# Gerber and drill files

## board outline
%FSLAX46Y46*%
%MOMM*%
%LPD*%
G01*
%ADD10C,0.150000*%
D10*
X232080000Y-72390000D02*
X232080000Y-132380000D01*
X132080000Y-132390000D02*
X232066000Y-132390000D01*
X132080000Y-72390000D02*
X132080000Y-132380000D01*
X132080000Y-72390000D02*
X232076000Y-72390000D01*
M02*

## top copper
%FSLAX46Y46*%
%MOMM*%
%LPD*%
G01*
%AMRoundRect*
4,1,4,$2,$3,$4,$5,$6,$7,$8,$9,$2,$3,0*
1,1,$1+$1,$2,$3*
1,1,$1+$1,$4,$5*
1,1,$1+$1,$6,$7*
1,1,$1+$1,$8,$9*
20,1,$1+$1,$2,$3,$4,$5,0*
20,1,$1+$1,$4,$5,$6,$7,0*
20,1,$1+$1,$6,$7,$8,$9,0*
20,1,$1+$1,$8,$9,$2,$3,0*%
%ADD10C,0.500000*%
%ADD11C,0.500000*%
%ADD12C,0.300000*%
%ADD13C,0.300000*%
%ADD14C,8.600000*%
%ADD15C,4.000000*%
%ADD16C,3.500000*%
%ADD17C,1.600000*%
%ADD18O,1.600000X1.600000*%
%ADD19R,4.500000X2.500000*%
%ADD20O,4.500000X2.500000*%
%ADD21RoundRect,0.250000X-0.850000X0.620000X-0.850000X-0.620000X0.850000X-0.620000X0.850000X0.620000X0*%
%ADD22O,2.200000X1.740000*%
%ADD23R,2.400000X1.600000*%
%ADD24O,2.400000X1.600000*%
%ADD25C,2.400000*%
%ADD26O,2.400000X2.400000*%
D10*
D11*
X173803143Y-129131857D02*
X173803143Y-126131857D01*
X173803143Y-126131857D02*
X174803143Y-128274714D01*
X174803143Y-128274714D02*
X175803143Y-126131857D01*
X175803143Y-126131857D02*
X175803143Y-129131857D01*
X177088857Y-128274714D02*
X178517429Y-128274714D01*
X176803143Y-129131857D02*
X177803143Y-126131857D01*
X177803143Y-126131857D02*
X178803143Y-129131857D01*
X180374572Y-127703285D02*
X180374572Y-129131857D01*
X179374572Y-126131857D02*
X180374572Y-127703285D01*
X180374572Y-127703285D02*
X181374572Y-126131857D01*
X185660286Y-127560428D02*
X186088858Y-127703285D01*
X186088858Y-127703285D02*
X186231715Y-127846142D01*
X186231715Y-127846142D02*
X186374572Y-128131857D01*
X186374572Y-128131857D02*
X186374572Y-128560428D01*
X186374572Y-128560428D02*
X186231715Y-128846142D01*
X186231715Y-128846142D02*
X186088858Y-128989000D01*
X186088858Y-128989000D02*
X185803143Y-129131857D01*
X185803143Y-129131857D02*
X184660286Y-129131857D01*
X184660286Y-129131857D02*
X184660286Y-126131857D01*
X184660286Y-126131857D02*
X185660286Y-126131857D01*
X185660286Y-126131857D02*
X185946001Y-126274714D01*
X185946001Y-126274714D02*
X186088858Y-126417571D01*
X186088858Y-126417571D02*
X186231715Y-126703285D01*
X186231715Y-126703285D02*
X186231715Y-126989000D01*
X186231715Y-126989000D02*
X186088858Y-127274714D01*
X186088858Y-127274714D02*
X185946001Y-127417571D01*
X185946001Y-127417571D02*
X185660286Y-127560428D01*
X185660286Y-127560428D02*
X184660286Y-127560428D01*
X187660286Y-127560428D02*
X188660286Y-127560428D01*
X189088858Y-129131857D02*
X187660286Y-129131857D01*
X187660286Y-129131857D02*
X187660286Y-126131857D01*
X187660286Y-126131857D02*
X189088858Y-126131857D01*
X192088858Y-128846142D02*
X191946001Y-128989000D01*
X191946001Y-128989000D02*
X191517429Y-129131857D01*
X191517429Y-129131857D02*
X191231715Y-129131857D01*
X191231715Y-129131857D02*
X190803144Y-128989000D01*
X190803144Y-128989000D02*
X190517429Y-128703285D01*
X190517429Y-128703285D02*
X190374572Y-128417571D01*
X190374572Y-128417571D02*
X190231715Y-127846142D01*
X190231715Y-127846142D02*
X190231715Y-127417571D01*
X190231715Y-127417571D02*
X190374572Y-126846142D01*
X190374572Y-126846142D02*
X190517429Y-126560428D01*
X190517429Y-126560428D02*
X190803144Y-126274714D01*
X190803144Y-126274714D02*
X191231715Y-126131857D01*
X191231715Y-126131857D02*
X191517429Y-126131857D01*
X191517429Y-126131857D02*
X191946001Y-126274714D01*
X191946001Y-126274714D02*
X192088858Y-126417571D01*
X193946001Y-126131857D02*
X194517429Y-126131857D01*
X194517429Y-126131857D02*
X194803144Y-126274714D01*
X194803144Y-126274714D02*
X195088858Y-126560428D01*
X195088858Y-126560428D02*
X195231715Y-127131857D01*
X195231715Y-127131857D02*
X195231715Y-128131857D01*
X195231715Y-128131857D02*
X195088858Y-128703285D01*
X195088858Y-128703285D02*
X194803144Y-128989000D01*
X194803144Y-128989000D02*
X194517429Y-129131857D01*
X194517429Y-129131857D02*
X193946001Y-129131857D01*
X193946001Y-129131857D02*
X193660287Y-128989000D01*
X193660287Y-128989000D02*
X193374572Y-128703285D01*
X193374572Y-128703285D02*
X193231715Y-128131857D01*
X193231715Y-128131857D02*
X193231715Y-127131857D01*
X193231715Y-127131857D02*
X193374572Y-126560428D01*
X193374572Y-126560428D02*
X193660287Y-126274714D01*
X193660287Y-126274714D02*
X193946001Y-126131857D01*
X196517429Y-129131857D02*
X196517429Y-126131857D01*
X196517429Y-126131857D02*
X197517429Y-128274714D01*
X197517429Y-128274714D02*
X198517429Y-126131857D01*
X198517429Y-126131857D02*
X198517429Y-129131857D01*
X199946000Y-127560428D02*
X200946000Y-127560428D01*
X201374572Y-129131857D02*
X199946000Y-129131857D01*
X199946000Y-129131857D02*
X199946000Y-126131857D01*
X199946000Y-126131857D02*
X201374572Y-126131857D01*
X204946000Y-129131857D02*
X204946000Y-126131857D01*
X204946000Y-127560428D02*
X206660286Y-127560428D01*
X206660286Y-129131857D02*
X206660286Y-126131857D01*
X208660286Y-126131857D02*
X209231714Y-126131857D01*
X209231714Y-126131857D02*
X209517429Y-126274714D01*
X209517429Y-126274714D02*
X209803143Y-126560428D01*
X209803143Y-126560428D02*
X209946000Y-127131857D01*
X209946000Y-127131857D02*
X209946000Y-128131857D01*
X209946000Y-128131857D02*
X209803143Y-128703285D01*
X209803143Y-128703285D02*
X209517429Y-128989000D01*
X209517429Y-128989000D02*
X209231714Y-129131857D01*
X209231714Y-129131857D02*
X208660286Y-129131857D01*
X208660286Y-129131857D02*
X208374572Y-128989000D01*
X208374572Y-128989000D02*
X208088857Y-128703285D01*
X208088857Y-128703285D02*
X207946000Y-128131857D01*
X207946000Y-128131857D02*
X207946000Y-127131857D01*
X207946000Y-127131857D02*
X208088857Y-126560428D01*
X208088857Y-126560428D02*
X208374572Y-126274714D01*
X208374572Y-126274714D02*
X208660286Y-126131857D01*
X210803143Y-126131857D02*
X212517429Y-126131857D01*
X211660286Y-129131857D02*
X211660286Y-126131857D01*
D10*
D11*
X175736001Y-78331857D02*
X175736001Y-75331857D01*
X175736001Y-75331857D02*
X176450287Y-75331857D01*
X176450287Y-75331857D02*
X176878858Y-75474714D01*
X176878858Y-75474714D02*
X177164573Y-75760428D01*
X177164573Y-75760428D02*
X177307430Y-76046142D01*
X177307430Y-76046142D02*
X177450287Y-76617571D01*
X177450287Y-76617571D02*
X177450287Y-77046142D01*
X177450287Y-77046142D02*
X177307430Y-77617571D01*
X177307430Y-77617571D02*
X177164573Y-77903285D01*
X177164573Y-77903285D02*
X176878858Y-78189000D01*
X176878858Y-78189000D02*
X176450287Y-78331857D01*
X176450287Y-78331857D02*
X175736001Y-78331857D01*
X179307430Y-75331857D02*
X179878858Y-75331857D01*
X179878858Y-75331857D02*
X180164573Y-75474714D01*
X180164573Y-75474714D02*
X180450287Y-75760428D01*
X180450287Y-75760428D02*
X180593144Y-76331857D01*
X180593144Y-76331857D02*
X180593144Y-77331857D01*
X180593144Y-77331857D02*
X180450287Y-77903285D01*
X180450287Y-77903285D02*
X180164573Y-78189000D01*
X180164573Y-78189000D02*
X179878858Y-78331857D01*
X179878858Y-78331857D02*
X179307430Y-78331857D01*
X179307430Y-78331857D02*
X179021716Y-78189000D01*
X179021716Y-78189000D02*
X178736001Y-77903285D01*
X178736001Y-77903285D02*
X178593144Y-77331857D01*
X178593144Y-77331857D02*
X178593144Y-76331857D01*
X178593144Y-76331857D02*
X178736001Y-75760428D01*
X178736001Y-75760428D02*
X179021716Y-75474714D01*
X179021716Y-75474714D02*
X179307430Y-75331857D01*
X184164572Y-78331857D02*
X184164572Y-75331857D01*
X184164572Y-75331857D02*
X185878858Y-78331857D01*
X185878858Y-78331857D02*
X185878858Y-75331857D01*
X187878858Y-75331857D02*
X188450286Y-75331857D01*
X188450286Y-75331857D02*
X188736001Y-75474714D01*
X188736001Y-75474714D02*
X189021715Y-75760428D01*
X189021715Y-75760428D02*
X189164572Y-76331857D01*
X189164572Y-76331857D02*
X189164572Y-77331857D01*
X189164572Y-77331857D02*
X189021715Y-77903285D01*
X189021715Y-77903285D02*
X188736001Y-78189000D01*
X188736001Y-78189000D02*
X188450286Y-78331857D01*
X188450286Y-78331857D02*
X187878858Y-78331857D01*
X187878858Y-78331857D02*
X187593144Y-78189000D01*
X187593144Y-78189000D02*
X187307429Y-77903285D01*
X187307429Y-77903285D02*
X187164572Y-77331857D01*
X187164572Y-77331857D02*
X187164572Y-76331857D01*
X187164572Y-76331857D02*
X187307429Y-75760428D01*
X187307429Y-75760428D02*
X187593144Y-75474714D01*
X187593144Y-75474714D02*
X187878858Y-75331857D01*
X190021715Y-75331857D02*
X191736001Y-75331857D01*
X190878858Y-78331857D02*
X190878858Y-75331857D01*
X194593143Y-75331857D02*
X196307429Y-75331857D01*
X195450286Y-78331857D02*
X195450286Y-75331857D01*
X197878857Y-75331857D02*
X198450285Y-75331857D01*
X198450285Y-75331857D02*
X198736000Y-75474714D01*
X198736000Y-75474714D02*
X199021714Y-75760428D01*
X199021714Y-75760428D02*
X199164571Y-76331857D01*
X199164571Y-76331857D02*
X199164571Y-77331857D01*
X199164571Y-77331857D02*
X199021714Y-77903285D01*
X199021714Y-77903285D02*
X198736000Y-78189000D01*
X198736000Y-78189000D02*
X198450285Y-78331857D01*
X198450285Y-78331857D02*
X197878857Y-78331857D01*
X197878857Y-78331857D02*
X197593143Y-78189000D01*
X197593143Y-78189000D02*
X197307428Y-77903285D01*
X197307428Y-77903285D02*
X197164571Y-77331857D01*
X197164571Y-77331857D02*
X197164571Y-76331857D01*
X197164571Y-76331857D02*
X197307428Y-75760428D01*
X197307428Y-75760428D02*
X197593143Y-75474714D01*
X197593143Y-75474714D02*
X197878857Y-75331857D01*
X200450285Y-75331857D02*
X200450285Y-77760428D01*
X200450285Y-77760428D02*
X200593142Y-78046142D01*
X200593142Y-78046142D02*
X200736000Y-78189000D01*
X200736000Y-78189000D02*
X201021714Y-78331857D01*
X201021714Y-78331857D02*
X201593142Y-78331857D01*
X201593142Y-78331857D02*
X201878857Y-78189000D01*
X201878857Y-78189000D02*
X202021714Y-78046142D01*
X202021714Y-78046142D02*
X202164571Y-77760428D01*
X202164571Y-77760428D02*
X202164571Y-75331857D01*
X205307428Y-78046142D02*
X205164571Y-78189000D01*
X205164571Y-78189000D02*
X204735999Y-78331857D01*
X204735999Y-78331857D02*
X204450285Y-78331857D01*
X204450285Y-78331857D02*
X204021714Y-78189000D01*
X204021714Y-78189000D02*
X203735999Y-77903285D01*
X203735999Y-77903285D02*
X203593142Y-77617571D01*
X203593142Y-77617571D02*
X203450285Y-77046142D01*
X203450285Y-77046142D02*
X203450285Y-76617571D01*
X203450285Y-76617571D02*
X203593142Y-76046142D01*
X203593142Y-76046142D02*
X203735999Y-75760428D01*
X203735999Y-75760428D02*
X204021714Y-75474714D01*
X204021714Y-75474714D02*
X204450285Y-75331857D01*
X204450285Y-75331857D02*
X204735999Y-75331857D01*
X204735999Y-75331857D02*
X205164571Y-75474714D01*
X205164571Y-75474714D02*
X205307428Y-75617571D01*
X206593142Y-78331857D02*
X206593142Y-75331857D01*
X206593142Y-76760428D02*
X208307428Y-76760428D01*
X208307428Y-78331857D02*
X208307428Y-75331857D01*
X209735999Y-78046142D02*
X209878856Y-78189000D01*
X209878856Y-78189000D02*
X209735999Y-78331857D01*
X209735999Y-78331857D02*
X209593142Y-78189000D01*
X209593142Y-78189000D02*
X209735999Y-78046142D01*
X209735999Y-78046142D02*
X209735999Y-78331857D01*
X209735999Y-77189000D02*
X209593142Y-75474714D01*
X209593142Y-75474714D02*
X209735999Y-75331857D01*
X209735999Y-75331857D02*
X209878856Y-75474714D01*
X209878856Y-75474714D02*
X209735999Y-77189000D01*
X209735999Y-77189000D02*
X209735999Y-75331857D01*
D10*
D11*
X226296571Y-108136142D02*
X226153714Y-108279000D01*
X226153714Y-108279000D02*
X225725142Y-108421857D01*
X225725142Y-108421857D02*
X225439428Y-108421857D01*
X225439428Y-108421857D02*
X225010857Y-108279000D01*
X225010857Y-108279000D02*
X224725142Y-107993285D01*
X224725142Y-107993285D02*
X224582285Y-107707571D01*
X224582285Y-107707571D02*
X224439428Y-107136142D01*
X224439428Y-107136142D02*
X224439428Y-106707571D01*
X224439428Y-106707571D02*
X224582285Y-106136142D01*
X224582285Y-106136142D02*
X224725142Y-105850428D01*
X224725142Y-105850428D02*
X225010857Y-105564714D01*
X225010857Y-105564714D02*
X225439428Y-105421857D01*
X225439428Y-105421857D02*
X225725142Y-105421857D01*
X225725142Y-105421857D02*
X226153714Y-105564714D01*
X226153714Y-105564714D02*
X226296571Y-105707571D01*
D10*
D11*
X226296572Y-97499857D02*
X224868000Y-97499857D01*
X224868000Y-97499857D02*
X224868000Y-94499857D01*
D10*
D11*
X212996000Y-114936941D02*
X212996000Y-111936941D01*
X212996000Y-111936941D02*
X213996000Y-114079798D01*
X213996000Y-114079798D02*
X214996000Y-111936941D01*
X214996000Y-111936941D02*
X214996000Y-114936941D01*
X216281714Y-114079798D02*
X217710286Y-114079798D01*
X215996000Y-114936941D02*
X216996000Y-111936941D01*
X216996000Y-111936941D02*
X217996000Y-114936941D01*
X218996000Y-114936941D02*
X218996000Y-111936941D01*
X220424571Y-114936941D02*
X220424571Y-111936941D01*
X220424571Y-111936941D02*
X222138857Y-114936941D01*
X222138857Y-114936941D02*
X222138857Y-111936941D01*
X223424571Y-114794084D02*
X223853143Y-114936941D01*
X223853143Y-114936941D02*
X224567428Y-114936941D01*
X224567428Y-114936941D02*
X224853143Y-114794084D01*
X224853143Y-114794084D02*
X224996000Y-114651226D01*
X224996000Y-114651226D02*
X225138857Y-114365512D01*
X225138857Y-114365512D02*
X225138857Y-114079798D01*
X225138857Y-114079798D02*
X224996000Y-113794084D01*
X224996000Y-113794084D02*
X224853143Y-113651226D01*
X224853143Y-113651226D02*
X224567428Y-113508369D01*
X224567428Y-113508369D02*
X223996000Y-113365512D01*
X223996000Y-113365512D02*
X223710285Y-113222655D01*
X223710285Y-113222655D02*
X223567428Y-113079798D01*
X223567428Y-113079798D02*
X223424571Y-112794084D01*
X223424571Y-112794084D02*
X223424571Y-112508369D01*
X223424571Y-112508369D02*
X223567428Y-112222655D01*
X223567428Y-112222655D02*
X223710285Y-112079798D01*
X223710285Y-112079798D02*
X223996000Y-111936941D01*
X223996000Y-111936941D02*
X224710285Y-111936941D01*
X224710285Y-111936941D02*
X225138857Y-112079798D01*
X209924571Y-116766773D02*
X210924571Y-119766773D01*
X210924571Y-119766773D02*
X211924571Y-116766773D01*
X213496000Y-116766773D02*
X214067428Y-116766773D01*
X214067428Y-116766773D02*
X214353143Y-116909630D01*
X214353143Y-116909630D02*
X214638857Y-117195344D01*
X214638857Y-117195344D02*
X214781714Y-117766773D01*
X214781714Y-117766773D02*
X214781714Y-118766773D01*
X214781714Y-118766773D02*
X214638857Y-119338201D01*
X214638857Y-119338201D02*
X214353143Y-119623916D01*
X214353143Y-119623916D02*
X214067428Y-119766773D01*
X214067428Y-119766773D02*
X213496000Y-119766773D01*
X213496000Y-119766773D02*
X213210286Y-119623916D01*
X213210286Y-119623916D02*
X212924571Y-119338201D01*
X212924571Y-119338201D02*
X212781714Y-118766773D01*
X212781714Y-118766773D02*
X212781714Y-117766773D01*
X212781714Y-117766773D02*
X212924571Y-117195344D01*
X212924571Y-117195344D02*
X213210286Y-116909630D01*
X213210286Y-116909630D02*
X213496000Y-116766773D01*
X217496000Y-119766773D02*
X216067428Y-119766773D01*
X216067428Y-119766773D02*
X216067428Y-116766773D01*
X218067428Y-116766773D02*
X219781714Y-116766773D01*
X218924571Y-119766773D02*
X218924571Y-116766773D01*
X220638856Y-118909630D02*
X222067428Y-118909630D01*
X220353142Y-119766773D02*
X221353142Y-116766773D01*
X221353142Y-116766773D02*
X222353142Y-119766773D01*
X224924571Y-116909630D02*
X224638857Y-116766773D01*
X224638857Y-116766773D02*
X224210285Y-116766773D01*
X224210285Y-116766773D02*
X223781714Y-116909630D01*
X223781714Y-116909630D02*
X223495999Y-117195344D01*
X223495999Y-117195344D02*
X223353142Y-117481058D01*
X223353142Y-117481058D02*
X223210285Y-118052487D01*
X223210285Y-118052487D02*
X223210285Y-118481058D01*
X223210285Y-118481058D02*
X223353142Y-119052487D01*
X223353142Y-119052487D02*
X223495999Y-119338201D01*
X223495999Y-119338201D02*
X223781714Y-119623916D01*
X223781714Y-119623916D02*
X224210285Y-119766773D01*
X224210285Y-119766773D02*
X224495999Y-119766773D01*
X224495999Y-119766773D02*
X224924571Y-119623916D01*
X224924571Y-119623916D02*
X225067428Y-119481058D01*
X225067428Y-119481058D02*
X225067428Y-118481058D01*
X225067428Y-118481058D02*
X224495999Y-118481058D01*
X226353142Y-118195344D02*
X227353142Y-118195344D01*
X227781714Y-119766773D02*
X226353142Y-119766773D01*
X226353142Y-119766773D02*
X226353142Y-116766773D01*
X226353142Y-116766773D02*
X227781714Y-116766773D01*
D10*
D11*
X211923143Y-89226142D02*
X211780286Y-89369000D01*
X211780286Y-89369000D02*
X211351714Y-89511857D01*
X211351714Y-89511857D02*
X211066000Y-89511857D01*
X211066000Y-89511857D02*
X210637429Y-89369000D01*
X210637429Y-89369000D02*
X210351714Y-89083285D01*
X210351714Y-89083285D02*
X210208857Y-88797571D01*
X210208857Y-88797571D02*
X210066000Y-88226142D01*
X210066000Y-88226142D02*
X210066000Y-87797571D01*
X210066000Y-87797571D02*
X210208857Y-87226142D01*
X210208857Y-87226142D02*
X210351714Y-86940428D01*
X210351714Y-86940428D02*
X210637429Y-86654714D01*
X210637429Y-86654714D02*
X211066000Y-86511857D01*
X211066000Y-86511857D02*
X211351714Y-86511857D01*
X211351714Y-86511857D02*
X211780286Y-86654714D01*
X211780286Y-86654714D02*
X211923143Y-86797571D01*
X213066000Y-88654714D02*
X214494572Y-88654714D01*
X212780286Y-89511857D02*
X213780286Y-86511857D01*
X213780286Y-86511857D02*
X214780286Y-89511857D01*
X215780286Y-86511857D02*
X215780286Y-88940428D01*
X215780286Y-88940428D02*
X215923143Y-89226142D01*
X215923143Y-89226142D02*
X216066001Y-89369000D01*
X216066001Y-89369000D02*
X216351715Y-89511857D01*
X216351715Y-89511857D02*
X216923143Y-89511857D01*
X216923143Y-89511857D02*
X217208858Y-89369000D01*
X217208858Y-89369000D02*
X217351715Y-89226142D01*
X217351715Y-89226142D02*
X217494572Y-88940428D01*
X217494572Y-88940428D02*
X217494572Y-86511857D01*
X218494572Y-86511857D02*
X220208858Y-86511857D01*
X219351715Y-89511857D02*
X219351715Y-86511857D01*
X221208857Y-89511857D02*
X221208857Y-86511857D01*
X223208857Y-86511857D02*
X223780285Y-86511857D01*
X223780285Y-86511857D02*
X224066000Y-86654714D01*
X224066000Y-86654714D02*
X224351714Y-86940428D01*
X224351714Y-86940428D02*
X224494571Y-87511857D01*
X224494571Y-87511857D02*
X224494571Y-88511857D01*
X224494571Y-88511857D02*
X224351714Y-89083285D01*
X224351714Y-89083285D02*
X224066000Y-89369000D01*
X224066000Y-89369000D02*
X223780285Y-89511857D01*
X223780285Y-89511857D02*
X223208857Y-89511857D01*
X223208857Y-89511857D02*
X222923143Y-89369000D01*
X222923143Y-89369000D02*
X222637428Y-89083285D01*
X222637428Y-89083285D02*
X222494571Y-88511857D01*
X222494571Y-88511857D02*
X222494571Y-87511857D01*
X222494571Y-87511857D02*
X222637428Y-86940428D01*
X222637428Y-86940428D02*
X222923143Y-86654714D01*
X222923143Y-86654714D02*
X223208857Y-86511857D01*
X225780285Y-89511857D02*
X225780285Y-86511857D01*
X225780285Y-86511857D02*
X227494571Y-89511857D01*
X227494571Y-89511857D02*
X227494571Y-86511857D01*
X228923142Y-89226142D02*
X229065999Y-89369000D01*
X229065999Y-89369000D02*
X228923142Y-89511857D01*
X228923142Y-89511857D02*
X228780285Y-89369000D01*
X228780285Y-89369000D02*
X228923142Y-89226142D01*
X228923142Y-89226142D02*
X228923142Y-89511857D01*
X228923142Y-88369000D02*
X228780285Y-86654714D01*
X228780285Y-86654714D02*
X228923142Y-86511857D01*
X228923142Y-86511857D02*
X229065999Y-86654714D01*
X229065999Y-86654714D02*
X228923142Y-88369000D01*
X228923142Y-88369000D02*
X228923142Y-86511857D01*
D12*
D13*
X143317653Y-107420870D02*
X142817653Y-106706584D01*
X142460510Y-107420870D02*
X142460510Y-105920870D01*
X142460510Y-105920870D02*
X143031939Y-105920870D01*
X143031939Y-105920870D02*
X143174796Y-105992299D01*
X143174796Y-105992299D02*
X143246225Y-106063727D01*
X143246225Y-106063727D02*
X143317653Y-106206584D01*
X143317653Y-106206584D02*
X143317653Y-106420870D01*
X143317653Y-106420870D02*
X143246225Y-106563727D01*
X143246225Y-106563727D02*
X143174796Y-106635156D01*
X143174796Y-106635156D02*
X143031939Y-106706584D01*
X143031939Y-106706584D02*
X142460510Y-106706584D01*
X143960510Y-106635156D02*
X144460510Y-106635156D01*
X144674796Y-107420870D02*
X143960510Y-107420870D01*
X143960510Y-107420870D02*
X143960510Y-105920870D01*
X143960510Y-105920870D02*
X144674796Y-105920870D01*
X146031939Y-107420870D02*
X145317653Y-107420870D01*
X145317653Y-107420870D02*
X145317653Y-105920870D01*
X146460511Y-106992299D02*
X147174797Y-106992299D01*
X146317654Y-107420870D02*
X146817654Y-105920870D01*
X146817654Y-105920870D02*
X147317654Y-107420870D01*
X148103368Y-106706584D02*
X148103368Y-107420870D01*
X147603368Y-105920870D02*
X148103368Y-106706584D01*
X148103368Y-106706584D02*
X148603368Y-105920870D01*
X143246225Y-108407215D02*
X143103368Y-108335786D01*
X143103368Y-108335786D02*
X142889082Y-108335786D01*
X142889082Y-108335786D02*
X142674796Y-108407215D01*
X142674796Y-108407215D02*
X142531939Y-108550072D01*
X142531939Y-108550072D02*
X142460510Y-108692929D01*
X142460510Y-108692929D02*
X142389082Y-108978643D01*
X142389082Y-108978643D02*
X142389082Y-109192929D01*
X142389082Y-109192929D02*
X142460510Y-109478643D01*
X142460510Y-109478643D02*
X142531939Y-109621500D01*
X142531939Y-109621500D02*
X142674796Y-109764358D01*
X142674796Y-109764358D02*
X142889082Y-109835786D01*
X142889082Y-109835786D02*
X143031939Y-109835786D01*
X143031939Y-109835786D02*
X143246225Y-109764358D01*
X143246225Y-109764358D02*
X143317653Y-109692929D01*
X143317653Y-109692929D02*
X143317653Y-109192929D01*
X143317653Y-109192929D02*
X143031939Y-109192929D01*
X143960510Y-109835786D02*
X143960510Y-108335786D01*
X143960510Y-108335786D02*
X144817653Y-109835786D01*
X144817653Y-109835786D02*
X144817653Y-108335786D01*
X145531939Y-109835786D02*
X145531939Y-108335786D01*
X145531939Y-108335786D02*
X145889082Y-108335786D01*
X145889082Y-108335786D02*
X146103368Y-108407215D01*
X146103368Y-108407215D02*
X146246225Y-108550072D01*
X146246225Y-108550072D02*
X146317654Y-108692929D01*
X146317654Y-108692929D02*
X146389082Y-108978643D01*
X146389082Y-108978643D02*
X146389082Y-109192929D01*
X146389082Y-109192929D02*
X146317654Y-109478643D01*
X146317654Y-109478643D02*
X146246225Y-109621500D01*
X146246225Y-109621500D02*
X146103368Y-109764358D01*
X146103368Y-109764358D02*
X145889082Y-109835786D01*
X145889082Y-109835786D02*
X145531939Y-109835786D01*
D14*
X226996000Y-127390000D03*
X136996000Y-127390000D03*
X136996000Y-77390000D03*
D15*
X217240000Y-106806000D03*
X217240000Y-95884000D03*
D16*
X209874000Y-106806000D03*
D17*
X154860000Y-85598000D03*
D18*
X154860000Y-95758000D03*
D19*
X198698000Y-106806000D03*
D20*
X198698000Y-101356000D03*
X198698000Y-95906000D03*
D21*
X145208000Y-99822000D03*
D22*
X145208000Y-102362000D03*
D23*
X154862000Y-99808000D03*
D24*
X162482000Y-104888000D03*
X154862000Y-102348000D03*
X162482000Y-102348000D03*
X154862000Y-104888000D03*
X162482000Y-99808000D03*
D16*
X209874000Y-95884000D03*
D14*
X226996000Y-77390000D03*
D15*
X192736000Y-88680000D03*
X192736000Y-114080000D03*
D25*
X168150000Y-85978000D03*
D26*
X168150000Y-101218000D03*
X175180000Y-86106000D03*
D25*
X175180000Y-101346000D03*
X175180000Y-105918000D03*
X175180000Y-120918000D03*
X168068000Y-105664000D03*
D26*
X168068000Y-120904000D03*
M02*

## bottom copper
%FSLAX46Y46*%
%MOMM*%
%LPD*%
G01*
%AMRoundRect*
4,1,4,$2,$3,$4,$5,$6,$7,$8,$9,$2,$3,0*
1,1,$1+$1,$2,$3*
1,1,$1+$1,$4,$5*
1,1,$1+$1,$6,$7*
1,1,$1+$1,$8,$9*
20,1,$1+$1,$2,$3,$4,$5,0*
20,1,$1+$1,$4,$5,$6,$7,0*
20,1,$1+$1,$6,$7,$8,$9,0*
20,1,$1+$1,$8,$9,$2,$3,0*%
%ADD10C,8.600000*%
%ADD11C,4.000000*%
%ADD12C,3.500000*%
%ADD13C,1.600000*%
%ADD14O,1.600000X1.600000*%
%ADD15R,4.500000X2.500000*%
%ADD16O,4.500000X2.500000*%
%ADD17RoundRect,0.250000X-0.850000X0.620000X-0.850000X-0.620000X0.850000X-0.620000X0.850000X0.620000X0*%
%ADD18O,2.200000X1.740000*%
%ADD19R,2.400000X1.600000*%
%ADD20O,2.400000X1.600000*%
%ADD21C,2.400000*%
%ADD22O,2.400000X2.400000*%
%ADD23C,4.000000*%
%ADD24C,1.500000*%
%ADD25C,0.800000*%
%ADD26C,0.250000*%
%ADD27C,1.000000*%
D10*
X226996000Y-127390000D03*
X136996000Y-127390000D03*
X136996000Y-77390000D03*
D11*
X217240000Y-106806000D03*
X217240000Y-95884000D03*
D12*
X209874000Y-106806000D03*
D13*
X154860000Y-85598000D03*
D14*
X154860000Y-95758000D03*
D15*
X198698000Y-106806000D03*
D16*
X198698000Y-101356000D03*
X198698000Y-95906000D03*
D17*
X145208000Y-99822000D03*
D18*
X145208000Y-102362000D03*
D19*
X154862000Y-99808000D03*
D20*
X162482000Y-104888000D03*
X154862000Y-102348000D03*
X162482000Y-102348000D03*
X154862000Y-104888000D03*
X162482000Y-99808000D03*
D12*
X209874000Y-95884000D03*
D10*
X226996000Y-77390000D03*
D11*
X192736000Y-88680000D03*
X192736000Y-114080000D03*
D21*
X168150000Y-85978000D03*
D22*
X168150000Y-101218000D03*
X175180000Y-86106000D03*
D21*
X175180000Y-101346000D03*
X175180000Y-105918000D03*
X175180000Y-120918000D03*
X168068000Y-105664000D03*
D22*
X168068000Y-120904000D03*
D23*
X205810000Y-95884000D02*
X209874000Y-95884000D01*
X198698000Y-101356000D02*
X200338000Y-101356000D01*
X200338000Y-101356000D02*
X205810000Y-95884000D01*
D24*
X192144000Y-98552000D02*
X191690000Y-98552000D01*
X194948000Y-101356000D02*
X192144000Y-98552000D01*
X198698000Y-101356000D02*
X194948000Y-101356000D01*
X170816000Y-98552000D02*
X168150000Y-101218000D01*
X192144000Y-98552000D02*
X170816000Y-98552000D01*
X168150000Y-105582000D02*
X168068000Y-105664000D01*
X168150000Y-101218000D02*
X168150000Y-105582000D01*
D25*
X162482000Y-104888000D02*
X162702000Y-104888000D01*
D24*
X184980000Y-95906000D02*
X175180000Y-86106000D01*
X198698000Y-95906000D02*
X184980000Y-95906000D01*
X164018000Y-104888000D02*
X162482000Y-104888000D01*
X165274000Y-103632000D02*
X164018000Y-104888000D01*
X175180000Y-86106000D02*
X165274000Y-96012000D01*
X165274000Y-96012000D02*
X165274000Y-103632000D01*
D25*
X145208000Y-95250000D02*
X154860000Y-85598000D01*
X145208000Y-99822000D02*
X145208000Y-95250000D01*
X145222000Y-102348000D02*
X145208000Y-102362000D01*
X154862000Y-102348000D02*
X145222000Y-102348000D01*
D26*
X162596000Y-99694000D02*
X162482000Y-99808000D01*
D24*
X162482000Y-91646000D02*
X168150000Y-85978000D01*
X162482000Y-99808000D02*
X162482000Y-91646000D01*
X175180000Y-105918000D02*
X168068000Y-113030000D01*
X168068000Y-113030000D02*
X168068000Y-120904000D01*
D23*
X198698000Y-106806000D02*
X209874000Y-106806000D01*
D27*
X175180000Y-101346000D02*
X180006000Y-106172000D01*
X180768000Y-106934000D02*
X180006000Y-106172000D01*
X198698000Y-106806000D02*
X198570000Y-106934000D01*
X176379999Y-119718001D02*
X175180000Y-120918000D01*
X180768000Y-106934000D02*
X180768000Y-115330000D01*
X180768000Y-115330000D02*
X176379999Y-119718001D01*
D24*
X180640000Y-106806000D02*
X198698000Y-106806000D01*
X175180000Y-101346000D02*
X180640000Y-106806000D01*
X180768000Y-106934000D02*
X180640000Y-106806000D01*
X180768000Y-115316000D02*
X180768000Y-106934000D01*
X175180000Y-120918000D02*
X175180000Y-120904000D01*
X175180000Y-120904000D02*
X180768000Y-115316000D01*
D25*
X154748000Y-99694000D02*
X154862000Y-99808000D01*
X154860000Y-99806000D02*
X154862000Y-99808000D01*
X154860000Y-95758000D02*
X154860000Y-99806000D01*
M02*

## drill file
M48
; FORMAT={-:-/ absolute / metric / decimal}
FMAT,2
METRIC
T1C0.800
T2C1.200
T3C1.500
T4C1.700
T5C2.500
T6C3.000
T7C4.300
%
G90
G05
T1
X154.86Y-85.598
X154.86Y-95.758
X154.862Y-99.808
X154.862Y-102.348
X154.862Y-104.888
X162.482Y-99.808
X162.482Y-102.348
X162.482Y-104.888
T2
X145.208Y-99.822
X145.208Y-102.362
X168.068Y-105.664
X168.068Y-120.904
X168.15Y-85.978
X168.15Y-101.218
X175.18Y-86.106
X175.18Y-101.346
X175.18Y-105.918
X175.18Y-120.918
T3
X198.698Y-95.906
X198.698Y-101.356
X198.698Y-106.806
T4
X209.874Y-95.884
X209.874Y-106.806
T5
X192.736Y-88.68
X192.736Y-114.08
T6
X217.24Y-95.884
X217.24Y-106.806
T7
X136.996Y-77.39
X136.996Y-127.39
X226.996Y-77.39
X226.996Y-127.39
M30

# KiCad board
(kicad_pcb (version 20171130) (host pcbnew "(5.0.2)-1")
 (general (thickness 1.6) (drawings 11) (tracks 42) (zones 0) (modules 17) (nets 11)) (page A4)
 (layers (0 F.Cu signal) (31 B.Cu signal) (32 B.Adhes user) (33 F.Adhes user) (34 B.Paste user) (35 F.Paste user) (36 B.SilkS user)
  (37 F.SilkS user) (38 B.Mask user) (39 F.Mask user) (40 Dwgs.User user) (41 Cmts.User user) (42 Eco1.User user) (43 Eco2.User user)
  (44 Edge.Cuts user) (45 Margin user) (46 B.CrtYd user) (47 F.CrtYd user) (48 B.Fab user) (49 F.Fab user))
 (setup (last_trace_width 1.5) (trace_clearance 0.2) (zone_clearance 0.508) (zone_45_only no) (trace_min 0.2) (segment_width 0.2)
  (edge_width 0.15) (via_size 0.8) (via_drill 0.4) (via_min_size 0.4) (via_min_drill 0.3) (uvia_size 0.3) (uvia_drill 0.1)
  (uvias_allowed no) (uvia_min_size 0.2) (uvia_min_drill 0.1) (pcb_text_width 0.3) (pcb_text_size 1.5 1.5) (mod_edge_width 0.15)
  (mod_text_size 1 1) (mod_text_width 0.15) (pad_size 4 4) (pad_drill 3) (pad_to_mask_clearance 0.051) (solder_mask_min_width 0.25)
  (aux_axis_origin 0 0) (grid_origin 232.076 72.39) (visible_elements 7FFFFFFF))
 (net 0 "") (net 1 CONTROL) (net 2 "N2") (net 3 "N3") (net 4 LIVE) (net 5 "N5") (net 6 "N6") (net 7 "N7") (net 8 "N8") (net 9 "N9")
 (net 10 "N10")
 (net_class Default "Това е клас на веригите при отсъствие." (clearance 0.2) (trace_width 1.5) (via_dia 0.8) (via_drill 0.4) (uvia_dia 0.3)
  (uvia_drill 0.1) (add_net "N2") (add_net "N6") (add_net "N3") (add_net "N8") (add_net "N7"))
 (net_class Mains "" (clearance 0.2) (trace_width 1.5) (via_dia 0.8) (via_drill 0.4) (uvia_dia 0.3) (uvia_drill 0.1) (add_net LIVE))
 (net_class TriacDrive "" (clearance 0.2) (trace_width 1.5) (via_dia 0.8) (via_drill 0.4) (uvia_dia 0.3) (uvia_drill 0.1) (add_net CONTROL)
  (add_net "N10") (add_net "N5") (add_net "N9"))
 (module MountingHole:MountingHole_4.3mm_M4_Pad (layer F.Cu) (at 226.996 127.39)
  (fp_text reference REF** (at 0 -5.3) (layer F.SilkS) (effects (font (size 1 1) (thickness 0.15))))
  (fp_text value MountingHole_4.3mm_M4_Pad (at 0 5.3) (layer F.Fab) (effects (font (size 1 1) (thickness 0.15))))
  (pad 1 thru_hole circle (at 0 0) (size 8.6 8.6) (drill 4.3) (layers *.Cu *.Mask)))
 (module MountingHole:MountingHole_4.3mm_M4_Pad (layer F.Cu) (at 136.996 127.39)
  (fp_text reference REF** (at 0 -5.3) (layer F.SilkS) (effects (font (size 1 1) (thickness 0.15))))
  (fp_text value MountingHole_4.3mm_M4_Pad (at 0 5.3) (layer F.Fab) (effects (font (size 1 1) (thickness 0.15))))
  (pad 1 thru_hole circle (at 0 0) (size 8.6 8.6) (drill 4.3) (layers *.Cu *.Mask)))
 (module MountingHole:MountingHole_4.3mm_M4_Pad (layer F.Cu) (at 136.996 77.39)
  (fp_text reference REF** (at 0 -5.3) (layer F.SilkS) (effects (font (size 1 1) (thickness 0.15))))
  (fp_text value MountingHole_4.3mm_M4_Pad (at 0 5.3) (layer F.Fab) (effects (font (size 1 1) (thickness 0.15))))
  (pad 1 thru_hole circle (at 0 0) (size 8.6 8.6) (drill 4.3) (layers *.Cu *.Mask)))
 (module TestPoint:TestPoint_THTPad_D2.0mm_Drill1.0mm (layer F.Cu) (at 217.24 106.806)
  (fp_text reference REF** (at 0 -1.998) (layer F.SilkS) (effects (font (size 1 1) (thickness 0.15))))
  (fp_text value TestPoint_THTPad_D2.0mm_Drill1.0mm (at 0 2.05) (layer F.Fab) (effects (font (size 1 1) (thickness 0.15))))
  (pad 1 thru_hole circle (at 0 0) (size 4 4) (drill 3) (layers *.Cu *.Mask)))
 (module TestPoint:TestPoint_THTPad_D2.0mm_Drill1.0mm (layer F.Cu) (at 217.24 95.884)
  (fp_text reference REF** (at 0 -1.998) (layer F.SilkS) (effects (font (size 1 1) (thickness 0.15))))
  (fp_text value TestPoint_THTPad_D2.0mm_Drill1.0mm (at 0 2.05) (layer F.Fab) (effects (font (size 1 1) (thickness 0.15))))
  (pad 1 thru_hole circle (at 0 0) (size 4 4) (drill 3) (layers *.Cu *.Mask)))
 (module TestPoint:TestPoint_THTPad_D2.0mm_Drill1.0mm (layer F.Cu) (at 209.874 106.806)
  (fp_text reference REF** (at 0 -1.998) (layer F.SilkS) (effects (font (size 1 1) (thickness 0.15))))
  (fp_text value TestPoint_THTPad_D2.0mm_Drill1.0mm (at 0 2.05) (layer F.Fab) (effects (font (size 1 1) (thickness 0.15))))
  (pad 1 thru_hole circle (at 0 0) (size 3.5 3.5) (drill 1.7) (layers *.Cu *.Mask) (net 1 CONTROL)))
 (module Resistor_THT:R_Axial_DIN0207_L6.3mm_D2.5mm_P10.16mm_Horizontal (layer F.Cu) (at 154.86 85.598 270)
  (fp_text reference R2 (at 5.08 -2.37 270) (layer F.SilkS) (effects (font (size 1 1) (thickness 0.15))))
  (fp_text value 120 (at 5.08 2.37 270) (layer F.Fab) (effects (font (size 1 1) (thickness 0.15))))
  (pad 1 thru_hole circle (at 0 0 270) (size 1.6 1.6) (drill 0.8) (layers *.Cu *.Mask) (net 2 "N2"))
  (pad 2 thru_hole oval (at 10.16 0 270) (size 1.6 1.6) (drill 0.8) (layers *.Cu *.Mask) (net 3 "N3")))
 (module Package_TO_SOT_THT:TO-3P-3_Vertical (layer F.Cu) (at 198.698 106.806 90)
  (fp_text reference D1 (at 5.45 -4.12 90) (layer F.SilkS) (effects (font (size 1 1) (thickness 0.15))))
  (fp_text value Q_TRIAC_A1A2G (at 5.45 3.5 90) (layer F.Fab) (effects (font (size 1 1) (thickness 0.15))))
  (pad 1 thru_hole rect (at 0 0 90) (size 2.5 4.5) (drill 1.5) (layers *.Cu *.Mask) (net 1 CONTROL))
  (pad 2 thru_hole oval (at 5.45 0 90) (size 2.5 4.5) (drill 1.5) (layers *.Cu *.Mask) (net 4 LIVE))
  (pad 3 thru_hole oval (at 10.9 0 90) (size 2.5 4.5) (drill 1.5) (layers *.Cu *.Mask) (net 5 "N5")))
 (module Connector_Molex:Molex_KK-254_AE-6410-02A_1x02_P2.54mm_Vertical (layer F.Cu) (at 145.208 99.822 270)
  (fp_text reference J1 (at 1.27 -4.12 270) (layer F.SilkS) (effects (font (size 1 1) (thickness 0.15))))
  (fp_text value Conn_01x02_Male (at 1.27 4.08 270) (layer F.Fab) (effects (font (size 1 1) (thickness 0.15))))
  (pad 1 thru_hole roundrect (at 0 0 270) (size 1.74 2.2) (drill 1.2) (layers *.Cu *.Mask) (roundrect_rratio 0.143678) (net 2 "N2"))
  (pad 2 thru_hole oval (at 2.54 0 270) (size 1.74 2.2) (drill 1.2) (layers *.Cu *.Mask) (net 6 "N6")))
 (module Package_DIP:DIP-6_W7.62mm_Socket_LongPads (layer F.Cu) (at 154.862 99.808)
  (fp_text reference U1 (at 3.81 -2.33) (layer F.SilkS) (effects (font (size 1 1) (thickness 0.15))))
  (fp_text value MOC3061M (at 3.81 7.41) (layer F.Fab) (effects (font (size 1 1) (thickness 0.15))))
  (pad 1 thru_hole rect (at 0 0) (size 2.4 1.6) (drill 0.8) (layers *.Cu *.Mask) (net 3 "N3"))
  (pad 4 thru_hole oval (at 7.62 5.08) (size 2.4 1.6) (drill 0.8) (layers *.Cu *.Mask) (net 5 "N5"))
  (pad 2 thru_hole oval (at 0 2.54) (size 2.4 1.6) (drill 0.8) (layers *.Cu *.Mask) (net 6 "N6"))
  (pad 5 thru_hole oval (at 7.62 2.54) (size 2.4 1.6) (drill 0.8) (layers *.Cu *.Mask) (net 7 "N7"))
  (pad 3 thru_hole oval (at 0 5.08) (size 2.4 1.6) (drill 0.8) (layers *.Cu *.Mask) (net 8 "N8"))
  (pad 6 thru_hole oval (at 7.62 0) (size 2.4 1.6) (drill 0.8) (layers *.Cu *.Mask) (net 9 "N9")))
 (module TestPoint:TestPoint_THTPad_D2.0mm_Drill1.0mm (layer F.Cu) (at 209.874 95.884)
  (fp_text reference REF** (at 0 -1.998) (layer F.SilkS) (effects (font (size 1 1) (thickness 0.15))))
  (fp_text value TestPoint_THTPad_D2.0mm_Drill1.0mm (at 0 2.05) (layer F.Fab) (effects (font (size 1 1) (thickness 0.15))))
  (pad 1 thru_hole circle (at 0 0) (size 3.5 3.5) (drill 1.7) (layers *.Cu *.Mask) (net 4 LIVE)))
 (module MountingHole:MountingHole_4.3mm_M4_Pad (layer F.Cu) (at 226.996 77.39)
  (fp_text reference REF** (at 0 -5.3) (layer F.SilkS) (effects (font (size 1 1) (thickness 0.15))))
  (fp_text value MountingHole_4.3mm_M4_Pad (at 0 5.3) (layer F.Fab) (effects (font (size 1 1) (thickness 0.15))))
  (pad 1 thru_hole circle (at 0 0) (size 8.6 8.6) (drill 4.3) (layers *.Cu *.Mask)))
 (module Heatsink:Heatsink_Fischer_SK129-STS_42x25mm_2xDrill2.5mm (layer F.Cu) (at 192.736 101.38 90)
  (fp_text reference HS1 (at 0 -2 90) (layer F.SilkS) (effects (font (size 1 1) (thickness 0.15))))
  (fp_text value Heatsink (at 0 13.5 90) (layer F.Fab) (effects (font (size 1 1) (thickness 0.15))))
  (pad 1 thru_hole circle (at 12.7 0 90) (size 4 4) (drill 2.5) (layers *.Cu *.Mask))
  (pad 1 thru_hole circle (at -12.7 0 270) (size 4 4) (drill 2.5) (layers *.Cu *.Mask)))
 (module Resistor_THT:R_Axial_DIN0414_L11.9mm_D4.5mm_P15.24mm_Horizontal (layer F.Cu) (at 168.15 85.978 270)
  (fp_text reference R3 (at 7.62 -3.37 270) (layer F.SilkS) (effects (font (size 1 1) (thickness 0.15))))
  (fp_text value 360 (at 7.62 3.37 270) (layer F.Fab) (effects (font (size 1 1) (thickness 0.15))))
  (pad 1 thru_hole circle (at 0 0 270) (size 2.4 2.4) (drill 1.2) (layers *.Cu *.Mask) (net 9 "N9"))
  (pad 2 thru_hole oval (at 15.24 0 270) (size 2.4 2.4) (drill 1.2) (layers *.Cu *.Mask) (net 4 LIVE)))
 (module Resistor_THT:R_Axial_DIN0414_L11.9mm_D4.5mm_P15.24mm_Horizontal (layer F.Cu) (at 175.18 101.346 90)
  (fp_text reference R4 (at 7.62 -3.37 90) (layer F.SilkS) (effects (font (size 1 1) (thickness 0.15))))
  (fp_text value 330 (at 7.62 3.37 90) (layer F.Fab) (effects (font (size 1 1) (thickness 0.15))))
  (pad 2 thru_hole oval (at 15.24 0 90) (size 2.4 2.4) (drill 1.2) (layers *.Cu *.Mask) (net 5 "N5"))
  (pad 1 thru_hole circle (at 0 0 90) (size 2.4 2.4) (drill 1.2) (layers *.Cu *.Mask) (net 1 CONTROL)))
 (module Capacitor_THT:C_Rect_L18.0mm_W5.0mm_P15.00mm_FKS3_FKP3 (layer F.Cu) (at 175.18 105.918 270)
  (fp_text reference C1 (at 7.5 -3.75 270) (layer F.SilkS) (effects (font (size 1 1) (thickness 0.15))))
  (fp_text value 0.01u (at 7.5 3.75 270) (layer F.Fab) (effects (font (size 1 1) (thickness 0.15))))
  (pad 1 thru_hole circle (at 0 0 270) (size 2.4 2.4) (drill 1.2) (layers *.Cu *.Mask) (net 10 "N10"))
  (pad 2 thru_hole circle (at 15 0 270) (size 2.4 2.4) (drill 1.2) (layers *.Cu *.Mask) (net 1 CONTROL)))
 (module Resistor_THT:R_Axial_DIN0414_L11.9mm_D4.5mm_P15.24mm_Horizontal (layer F.Cu) (at 168.068 105.664 270)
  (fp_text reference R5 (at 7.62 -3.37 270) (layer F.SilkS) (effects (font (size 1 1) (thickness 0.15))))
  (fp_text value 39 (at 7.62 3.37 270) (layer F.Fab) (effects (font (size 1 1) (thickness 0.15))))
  (pad 1 thru_hole circle (at 0 0 270) (size 2.4 2.4) (drill 1.2) (layers *.Cu *.Mask) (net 4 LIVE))
  (pad 2 thru_hole oval (at 15.24 0 270) (size 2.4 2.4) (drill 1.2) (layers *.Cu *.Mask) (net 10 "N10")))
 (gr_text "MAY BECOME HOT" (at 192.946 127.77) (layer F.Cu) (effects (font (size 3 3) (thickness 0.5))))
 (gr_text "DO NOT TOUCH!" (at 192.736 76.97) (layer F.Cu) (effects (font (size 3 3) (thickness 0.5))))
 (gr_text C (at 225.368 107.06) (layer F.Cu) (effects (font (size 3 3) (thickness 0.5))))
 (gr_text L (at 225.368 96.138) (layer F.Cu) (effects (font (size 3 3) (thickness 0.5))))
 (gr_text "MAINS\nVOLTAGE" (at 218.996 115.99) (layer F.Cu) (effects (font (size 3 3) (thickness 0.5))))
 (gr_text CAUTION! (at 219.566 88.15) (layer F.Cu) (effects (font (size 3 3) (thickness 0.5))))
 (gr_line (start 232.08 72.39) (end 232.08 132.38) (layer Edge.Cuts) (width 0.15))
 (gr_line (start 132.08 132.39) (end 232.066 132.39) (layer Edge.Cuts) (width 0.15))
 (gr_line (start 132.08 72.39) (end 132.08 132.38) (layer Edge.Cuts) (width 0.15))
 (gr_line (start 132.08 72.39) (end 232.076 72.39) (layer Edge.Cuts) (width 0.15))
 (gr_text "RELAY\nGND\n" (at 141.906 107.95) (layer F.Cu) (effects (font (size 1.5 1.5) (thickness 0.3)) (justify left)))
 (segment (start 205.81 95.884) (end 209.874 95.884) (width 4) (layer B.Cu) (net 4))
 (segment (start 198.698 101.356) (end 200.338 101.356) (width 4) (layer B.Cu) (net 4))
 (segment (start 200.338 101.356) (end 205.81 95.884) (width 4) (layer B.Cu) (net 4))
 (segment (start 192.144 98.552) (end 191.69 98.552) (width 1.5) (layer B.Cu) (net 4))
 (segment (start 194.948 101.356) (end 192.144 98.552) (width 1.5) (layer B.Cu) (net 4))
 (segment (start 198.698 101.356) (end 194.948 101.356) (width 1.5) (layer B.Cu) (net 4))
 (segment (start 170.816 98.552) (end 168.15 101.218) (width 1.5) (layer B.Cu) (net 4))
 (segment (start 192.144 98.552) (end 170.816 98.552) (width 1.5) (layer B.Cu) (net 4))
 (segment (start 168.15 105.582) (end 168.068 105.664) (width 1.5) (layer B.Cu) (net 4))
 (segment (start 168.15 101.218) (end 168.15 105.582) (width 1.5) (layer B.Cu) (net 4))
 (segment (start 162.482 104.888) (end 162.702 104.888) (width 0.8) (layer B.Cu) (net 5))
 (segment (start 184.98 95.906) (end 175.18 86.106) (width 1.5) (layer B.Cu) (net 5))
 (segment (start 198.698 95.906) (end 184.98 95.906) (width 1.5) (layer B.Cu) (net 5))
 (segment (start 164.018 104.888) (end 162.482 104.888) (width 1.5) (layer B.Cu) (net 5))
 (segment (start 165.274 103.632) (end 164.018 104.888) (width 1.5) (layer B.Cu) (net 5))
 (segment (start 175.18 86.106) (end 165.274 96.012) (width 1.5) (layer B.Cu) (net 5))
 (segment (start 165.274 96.012) (end 165.274 103.632) (width 1.5) (layer B.Cu) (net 5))
 (segment (start 145.208 95.25) (end 154.86 85.598) (width 0.8) (layer B.Cu) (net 2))
 (segment (start 145.208 99.822) (end 145.208 95.25) (width 0.8) (layer B.Cu) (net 2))
 (segment (start 145.222 102.348) (end 145.208 102.362) (width 0.8) (layer B.Cu) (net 6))
 (segment (start 154.862 102.348) (end 145.222 102.348) (width 0.8) (layer B.Cu) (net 6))
 (segment (start 162.596 99.694) (end 162.482 99.808) (width 0.25) (layer B.Cu) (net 9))
 (segment (start 162.482 91.646) (end 168.15 85.978) (width 1.5) (layer B.Cu) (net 9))
 (segment (start 162.482 99.808) (end 162.482 91.646) (width 1.5) (layer B.Cu) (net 9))
 (segment (start 175.18 105.918) (end 168.068 113.03) (width 1.5) (layer B.Cu) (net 10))
 (segment (start 168.068 113.03) (end 168.068 120.904) (width 1.5) (layer B.Cu) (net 10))
 (segment (start 198.698 106.806) (end 209.874 106.806) (width 4) (layer B.Cu) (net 1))
 (segment (start 175.18 101.346) (end 180.006 106.172) (width 1) (layer B.Cu) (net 1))
 (segment (start 180.768 106.934) (end 180.006 106.172) (width 1) (layer B.Cu) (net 1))
 (segment (start 198.698 106.806) (end 198.57 106.934) (width 1) (layer B.Cu) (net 1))
 (segment (start 176.379999 119.718001) (end 175.18 120.918) (width 1) (layer B.Cu) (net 1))
 (segment (start 180.768 106.934) (end 180.768 115.33) (width 1) (layer B.Cu) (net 1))
 (segment (start 180.768 115.33) (end 176.379999 119.718001) (width 1) (layer B.Cu) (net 1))
 (segment (start 180.64 106.806) (end 198.698 106.806) (width 1.5) (layer B.Cu) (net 1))
 (segment (start 175.18 101.346) (end 180.64 106.806) (width 1.5) (layer B.Cu) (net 1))
 (segment (start 180.768 106.934) (end 180.64 106.806) (width 1.5) (layer B.Cu) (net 1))
 (segment (start 180.768 115.316) (end 180.768 106.934) (width 1.5) (layer B.Cu) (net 1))
 (segment (start 175.18 120.918) (end 175.18 120.904) (width 1.5) (layer B.Cu) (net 1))
 (segment (start 175.18 120.904) (end 180.768 115.316) (width 1.5) (layer B.Cu) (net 1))
 (segment (start 154.748 99.694) (end 154.862 99.808) (width 0.8) (layer B.Cu) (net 3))
 (segment (start 154.86 99.806) (end 154.862 99.808) (width 0.8) (layer B.Cu) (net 3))
 (segment (start 154.86 95.758) (end 154.86 99.806) (width 0.8) (layer B.Cu) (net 3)))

